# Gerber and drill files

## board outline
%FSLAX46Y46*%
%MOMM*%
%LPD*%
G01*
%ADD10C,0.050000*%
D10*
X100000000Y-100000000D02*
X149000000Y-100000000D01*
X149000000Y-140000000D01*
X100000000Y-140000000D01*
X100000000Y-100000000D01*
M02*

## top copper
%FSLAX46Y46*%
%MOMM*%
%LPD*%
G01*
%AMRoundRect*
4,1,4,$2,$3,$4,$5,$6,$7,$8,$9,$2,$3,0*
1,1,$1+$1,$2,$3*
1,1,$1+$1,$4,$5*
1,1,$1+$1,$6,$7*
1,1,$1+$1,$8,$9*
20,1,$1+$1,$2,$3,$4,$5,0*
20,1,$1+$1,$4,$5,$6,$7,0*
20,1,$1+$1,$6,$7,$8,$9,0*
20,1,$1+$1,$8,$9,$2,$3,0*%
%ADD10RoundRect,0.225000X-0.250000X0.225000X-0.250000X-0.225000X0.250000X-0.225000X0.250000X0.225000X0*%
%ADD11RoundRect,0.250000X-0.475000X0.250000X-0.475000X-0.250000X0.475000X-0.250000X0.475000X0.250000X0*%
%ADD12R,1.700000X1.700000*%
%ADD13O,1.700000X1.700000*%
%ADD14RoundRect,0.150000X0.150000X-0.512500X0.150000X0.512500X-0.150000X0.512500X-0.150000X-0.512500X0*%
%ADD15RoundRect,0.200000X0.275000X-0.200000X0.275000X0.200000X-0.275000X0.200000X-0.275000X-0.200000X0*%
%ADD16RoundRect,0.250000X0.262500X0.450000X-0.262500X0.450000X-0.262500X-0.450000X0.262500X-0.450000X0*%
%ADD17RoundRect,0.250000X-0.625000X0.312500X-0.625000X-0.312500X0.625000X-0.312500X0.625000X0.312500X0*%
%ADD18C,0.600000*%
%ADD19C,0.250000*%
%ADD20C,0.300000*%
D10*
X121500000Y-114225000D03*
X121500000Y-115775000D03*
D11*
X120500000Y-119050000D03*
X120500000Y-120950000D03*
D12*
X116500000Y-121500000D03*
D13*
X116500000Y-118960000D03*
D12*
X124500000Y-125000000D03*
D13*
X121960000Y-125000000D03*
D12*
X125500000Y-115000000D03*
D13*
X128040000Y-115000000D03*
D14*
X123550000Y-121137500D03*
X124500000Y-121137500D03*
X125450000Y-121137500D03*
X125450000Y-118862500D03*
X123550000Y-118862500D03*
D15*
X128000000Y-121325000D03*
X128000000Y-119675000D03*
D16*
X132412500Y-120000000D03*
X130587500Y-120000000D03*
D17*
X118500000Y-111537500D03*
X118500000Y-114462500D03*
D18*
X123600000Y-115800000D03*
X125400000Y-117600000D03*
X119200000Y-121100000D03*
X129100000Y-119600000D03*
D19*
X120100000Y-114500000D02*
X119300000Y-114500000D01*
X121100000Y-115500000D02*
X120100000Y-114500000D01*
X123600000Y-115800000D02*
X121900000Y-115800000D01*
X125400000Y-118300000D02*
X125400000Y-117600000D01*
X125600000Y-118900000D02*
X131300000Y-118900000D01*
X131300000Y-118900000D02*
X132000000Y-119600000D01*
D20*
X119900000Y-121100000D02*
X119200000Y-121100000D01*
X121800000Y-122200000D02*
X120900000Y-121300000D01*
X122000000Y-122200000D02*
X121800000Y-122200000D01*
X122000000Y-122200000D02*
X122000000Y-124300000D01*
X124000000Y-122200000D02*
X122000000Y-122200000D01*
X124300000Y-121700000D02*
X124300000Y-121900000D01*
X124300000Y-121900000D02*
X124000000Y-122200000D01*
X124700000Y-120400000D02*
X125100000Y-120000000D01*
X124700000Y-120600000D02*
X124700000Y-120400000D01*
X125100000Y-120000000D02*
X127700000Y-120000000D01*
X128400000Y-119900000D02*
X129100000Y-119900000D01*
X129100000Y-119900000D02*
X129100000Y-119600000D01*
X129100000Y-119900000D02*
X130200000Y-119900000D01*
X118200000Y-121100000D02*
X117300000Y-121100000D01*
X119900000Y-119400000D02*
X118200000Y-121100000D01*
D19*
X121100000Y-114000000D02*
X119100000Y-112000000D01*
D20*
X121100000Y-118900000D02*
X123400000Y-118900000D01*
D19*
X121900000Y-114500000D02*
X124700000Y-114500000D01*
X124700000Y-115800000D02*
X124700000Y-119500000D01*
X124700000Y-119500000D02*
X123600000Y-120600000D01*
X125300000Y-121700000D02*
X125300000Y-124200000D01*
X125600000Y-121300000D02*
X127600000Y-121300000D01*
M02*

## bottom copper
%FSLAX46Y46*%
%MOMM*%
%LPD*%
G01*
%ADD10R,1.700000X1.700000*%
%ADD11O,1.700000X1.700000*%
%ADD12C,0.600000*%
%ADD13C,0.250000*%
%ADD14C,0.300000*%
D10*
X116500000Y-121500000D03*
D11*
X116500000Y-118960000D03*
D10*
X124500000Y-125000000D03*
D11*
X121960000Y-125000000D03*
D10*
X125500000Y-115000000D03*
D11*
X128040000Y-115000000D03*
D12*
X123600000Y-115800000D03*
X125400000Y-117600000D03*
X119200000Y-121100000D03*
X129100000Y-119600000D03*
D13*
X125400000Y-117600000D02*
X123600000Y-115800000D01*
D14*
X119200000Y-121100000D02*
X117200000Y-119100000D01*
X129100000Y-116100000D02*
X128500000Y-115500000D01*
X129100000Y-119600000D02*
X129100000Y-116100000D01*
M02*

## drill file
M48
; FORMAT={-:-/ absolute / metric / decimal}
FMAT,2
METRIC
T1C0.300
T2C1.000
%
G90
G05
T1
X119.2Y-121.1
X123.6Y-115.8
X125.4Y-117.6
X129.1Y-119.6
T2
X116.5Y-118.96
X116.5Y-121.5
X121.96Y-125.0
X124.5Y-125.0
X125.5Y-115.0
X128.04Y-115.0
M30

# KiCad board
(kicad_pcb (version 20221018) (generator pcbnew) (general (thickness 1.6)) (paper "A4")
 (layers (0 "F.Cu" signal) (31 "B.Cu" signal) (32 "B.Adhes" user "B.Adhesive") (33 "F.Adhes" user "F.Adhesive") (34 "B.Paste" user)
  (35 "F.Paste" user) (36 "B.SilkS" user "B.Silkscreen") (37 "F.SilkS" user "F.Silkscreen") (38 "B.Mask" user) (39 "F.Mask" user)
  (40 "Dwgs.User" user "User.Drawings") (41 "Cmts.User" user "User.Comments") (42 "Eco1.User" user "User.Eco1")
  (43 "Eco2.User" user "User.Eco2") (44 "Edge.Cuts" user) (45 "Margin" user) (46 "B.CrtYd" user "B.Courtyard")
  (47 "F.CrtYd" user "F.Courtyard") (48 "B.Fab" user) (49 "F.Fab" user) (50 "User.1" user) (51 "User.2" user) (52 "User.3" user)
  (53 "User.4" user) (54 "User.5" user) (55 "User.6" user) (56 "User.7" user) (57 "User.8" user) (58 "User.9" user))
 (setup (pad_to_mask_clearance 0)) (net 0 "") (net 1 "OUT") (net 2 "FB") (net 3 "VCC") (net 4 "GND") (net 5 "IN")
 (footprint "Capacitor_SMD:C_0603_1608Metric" (layer "F.Cu") (at 121.5 115 -90)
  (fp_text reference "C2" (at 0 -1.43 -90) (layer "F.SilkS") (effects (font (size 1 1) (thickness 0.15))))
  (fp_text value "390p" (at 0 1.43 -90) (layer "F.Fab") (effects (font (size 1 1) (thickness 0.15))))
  (pad "1" smd roundrect (at -0.775 0 270) (size 0.9 0.95) (layers "F.Cu" "F.Paste" "F.Mask") (roundrect_rratio 0.25) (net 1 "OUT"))
  (pad "2" smd roundrect (at 0.775 0 270) (size 0.9 0.95) (layers "F.Cu" "F.Paste" "F.Mask") (roundrect_rratio 0.25) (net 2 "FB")))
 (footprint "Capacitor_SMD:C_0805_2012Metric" (layer "F.Cu") (at 120.5 120 -90)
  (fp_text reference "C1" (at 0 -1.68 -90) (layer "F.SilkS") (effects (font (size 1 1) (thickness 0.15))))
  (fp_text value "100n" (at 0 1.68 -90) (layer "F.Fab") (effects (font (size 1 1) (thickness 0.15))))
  (pad "1" smd roundrect (at -0.95 0 270) (size 1 1.45) (layers "F.Cu" "F.Paste" "F.Mask") (roundrect_rratio 0.25) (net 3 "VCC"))
  (pad "2" smd roundrect (at 0.95 0 270) (size 1 1.45) (layers "F.Cu" "F.Paste" "F.Mask") (roundrect_rratio 0.25) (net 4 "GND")))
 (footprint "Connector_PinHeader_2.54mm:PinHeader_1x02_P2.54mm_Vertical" (layer "F.Cu") (at 116.5 121.5 180)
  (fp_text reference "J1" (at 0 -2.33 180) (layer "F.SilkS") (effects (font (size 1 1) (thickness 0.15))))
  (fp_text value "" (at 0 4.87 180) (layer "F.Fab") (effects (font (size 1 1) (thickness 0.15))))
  (pad "1" thru_hole rect (at 0 0 180) (size 1.7 1.7) (drill 1) (layers "*.Cu" "*.Mask") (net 3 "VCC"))
  (pad "2" thru_hole oval (at 0 2.54 180) (size 1.7 1.7) (drill 1) (layers "*.Cu" "*.Mask") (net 4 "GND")))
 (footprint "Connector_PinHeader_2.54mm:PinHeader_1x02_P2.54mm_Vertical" (layer "F.Cu") (at 124.5 125 -90)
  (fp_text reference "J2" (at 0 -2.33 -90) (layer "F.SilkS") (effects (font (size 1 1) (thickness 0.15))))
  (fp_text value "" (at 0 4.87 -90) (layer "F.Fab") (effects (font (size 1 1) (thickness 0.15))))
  (pad "1" thru_hole rect (at 0 0 270) (size 1.7 1.7) (drill 1) (layers "*.Cu" "*.Mask") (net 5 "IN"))
  (pad "2" thru_hole oval (at 0 2.54 270) (size 1.7 1.7) (drill 1) (layers "*.Cu" "*.Mask") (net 4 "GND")))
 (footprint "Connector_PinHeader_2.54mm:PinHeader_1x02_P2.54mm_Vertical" (layer "F.Cu") (at 125.5 115 90)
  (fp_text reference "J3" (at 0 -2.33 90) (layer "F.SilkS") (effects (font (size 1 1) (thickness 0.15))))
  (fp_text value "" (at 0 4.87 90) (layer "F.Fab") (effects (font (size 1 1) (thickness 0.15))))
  (pad "1" thru_hole rect (at 0 0 90) (size 1.7 1.7) (drill 1) (layers "*.Cu" "*.Mask") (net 1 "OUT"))
  (pad "2" thru_hole oval (at 0 2.54 90) (size 1.7 1.7) (drill 1) (layers "*.Cu" "*.Mask") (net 4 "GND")))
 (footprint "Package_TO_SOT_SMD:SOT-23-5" (layer "F.Cu") (at 124.5 120 90)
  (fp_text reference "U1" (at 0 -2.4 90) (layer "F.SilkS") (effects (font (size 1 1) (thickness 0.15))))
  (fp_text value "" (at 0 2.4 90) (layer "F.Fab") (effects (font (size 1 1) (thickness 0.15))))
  (pad "1" smd roundrect (at -1.1375 -0.95 90) (size 1.325 0.6) (layers "F.Cu" "F.Paste" "F.Mask") (roundrect_rratio 0.25) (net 1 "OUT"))
  (pad "2" smd roundrect (at -1.1375 0 90) (size 1.325 0.6) (layers "F.Cu" "F.Paste" "F.Mask") (roundrect_rratio 0.25) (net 4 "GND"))
  (pad "3" smd roundrect (at -1.1375 0.95 90) (size 1.325 0.6) (layers "F.Cu" "F.Paste" "F.Mask") (roundrect_rratio 0.25) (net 5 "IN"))
  (pad "4" smd roundrect (at 1.1375 0.95 90) (size 1.325 0.6) (layers "F.Cu" "F.Paste" "F.Mask") (roundrect_rratio 0.25) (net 2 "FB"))
  (pad "5" smd roundrect (at 1.1375 -0.95 90) (size 1.325 0.6) (layers "F.Cu" "F.Paste" "F.Mask") (roundrect_rratio 0.25) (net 3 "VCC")))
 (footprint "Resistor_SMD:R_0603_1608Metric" (layer "F.Cu") (at 128 120.5 90)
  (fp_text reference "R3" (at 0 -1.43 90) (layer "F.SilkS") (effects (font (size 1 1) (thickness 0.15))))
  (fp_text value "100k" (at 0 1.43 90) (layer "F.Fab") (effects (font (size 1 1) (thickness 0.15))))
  (pad "1" smd roundrect (at -0.825 0 90) (size 0.8 0.95) (layers "F.Cu" "F.Paste" "F.Mask") (roundrect_rratio 0.25) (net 5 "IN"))
  (pad "2" smd roundrect (at 0.825 0 90) (size 0.8 0.95) (layers "F.Cu" "F.Paste" "F.Mask") (roundrect_rratio 0.25) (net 4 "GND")))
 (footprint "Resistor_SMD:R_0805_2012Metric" (layer "F.Cu") (at 131.5 120 180)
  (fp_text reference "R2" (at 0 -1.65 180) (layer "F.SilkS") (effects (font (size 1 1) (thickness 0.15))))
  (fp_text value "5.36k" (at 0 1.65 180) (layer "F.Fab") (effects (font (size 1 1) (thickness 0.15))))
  (pad "1" smd roundrect (at -0.9125 0 180) (size 1.025 1.4) (layers "F.Cu" "F.Paste" "F.Mask") (roundrect_rratio 0.243902) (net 2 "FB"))
  (pad "2" smd roundrect (at 0.9125 0 180) (size 1.025 1.4) (layers "F.Cu" "F.Paste" "F.Mask") (roundrect_rratio 0.243902) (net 4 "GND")))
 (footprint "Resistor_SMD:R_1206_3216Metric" (layer "F.Cu") (at 118.5 113 -90)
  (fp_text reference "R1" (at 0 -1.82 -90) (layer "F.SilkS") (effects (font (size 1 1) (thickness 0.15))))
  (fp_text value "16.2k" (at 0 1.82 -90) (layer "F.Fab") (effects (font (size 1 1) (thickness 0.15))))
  (pad "1" smd roundrect (at -1.4625 0 270) (size 1.125 1.75) (layers "F.Cu" "F.Paste" "F.Mask") (roundrect_rratio 0.222222) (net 1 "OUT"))
  (pad "2" smd roundrect (at 1.4625 0 270) (size 1.125 1.75) (layers "F.Cu" "F.Paste" "F.Mask") (roundrect_rratio 0.222222) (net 2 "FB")))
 (gr_rect (start 100 100) (end 149 140) (stroke (width 0.05) (type default)) (fill none) (layer "Edge.Cuts"))
 (segment (start 120.1 114.5) (end 119.3 114.5) (width 0.25) (layer "F.Cu") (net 2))
 (segment (start 121.1 115.5) (end 120.1 114.5) (width 0.25) (layer "F.Cu") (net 2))
 (segment (start 123.6 115.8) (end 121.9 115.8) (width 0.25) (layer "F.Cu") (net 2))
 (segment (start 125.4 118.3) (end 125.4 117.6) (width 0.25) (layer "F.Cu") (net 2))
 (segment (start 125.6 118.9) (end 131.3 118.9) (width 0.25) (layer "F.Cu") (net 2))
 (segment (start 131.3 118.9) (end 132 119.6) (width 0.25) (layer "F.Cu") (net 2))
 (via (at 123.6 115.8) (size 0.6) (drill 0.3) (layers "F.Cu" "B.Cu") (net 2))
 (via (at 125.4 117.6) (size 0.6) (drill 0.3) (layers "F.Cu" "B.Cu") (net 2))
 (segment (start 119.9 121.1) (end 119.2 121.1) (width 0.3) (layer "F.Cu") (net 4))
 (segment (start 121.8 122.2) (end 120.9 121.3) (width 0.3) (layer "F.Cu") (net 4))
 (segment (start 122 122.2) (end 121.8 122.2) (width 0.3) (layer "F.Cu") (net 4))
 (segment (start 122 122.2) (end 122 124.3) (width 0.3) (layer "F.Cu") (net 4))
 (segment (start 124 122.2) (end 122 122.2) (width 0.3) (layer "F.Cu") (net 4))
 (segment (start 124.3 121.7) (end 124.3 121.9) (width 0.3) (layer "F.Cu") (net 4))
 (segment (start 124.3 121.9) (end 124 122.2) (width 0.3) (layer "F.Cu") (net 4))
 (segment (start 124.7 120.4) (end 125.1 120) (width 0.3) (layer "F.Cu") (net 4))
 (segment (start 124.7 120.6) (end 124.7 120.4) (width 0.3) (layer "F.Cu") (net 4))
 (segment (start 125.1 120) (end 127.7 120) (width 0.3) (layer "F.Cu") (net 4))
 (segment (start 125.4 117.6) (end 123.6 115.8) (width 0.25) (layer "B.Cu") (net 2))
 (segment (start 128.4 119.9) (end 129.1 119.9) (width 0.3) (layer "F.Cu") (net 4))
 (segment (start 129.1 119.9) (end 129.1 119.6) (width 0.3) (layer "F.Cu") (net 4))
 (segment (start 129.1 119.9) (end 130.2 119.9) (width 0.3) (layer "F.Cu") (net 4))
 (via (at 119.2 121.1) (size 0.6) (drill 0.3) (layers "F.Cu" "B.Cu") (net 4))
 (via (at 129.1 119.6) (size 0.6) (drill 0.3) (layers "F.Cu" "B.Cu") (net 4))
 (segment (start 118.2 121.1) (end 117.3 121.1) (width 0.3) (layer "F.Cu") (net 3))
 (segment (start 119.2 121.1) (end 117.2 119.1) (width 0.3) (layer "B.Cu") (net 4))
 (segment (start 119.9 119.4) (end 118.2 121.1) (width 0.3) (layer "F.Cu") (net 3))
 (segment (start 121.1 114) (end 119.1 112) (width 0.25) (layer "F.Cu") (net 1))
 (segment (start 121.1 118.9) (end 123.4 118.9) (width 0.3) (layer "F.Cu") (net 3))
 (segment (start 121.9 114.5) (end 124.7 114.5) (width 0.25) (layer "F.Cu") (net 1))
 (segment (start 124.7 115.8) (end 124.7 119.5) (width 0.25) (layer "F.Cu") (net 1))
 (segment (start 124.7 119.5) (end 123.6 120.6) (width 0.25) (layer "F.Cu") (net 1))
 (segment (start 125.3 121.7) (end 125.3 124.2) (width 0.25) (layer "F.Cu") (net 5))
 (segment (start 125.6 121.3) (end 127.6 121.3) (width 0.25) (layer "F.Cu") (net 5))
 (segment (start 129.1 116.1) (end 128.5 115.5) (width 0.3) (layer "B.Cu") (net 4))
 (segment (start 129.1 119.6) (end 129.1 116.1) (width 0.3) (layer "B.Cu") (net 4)))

